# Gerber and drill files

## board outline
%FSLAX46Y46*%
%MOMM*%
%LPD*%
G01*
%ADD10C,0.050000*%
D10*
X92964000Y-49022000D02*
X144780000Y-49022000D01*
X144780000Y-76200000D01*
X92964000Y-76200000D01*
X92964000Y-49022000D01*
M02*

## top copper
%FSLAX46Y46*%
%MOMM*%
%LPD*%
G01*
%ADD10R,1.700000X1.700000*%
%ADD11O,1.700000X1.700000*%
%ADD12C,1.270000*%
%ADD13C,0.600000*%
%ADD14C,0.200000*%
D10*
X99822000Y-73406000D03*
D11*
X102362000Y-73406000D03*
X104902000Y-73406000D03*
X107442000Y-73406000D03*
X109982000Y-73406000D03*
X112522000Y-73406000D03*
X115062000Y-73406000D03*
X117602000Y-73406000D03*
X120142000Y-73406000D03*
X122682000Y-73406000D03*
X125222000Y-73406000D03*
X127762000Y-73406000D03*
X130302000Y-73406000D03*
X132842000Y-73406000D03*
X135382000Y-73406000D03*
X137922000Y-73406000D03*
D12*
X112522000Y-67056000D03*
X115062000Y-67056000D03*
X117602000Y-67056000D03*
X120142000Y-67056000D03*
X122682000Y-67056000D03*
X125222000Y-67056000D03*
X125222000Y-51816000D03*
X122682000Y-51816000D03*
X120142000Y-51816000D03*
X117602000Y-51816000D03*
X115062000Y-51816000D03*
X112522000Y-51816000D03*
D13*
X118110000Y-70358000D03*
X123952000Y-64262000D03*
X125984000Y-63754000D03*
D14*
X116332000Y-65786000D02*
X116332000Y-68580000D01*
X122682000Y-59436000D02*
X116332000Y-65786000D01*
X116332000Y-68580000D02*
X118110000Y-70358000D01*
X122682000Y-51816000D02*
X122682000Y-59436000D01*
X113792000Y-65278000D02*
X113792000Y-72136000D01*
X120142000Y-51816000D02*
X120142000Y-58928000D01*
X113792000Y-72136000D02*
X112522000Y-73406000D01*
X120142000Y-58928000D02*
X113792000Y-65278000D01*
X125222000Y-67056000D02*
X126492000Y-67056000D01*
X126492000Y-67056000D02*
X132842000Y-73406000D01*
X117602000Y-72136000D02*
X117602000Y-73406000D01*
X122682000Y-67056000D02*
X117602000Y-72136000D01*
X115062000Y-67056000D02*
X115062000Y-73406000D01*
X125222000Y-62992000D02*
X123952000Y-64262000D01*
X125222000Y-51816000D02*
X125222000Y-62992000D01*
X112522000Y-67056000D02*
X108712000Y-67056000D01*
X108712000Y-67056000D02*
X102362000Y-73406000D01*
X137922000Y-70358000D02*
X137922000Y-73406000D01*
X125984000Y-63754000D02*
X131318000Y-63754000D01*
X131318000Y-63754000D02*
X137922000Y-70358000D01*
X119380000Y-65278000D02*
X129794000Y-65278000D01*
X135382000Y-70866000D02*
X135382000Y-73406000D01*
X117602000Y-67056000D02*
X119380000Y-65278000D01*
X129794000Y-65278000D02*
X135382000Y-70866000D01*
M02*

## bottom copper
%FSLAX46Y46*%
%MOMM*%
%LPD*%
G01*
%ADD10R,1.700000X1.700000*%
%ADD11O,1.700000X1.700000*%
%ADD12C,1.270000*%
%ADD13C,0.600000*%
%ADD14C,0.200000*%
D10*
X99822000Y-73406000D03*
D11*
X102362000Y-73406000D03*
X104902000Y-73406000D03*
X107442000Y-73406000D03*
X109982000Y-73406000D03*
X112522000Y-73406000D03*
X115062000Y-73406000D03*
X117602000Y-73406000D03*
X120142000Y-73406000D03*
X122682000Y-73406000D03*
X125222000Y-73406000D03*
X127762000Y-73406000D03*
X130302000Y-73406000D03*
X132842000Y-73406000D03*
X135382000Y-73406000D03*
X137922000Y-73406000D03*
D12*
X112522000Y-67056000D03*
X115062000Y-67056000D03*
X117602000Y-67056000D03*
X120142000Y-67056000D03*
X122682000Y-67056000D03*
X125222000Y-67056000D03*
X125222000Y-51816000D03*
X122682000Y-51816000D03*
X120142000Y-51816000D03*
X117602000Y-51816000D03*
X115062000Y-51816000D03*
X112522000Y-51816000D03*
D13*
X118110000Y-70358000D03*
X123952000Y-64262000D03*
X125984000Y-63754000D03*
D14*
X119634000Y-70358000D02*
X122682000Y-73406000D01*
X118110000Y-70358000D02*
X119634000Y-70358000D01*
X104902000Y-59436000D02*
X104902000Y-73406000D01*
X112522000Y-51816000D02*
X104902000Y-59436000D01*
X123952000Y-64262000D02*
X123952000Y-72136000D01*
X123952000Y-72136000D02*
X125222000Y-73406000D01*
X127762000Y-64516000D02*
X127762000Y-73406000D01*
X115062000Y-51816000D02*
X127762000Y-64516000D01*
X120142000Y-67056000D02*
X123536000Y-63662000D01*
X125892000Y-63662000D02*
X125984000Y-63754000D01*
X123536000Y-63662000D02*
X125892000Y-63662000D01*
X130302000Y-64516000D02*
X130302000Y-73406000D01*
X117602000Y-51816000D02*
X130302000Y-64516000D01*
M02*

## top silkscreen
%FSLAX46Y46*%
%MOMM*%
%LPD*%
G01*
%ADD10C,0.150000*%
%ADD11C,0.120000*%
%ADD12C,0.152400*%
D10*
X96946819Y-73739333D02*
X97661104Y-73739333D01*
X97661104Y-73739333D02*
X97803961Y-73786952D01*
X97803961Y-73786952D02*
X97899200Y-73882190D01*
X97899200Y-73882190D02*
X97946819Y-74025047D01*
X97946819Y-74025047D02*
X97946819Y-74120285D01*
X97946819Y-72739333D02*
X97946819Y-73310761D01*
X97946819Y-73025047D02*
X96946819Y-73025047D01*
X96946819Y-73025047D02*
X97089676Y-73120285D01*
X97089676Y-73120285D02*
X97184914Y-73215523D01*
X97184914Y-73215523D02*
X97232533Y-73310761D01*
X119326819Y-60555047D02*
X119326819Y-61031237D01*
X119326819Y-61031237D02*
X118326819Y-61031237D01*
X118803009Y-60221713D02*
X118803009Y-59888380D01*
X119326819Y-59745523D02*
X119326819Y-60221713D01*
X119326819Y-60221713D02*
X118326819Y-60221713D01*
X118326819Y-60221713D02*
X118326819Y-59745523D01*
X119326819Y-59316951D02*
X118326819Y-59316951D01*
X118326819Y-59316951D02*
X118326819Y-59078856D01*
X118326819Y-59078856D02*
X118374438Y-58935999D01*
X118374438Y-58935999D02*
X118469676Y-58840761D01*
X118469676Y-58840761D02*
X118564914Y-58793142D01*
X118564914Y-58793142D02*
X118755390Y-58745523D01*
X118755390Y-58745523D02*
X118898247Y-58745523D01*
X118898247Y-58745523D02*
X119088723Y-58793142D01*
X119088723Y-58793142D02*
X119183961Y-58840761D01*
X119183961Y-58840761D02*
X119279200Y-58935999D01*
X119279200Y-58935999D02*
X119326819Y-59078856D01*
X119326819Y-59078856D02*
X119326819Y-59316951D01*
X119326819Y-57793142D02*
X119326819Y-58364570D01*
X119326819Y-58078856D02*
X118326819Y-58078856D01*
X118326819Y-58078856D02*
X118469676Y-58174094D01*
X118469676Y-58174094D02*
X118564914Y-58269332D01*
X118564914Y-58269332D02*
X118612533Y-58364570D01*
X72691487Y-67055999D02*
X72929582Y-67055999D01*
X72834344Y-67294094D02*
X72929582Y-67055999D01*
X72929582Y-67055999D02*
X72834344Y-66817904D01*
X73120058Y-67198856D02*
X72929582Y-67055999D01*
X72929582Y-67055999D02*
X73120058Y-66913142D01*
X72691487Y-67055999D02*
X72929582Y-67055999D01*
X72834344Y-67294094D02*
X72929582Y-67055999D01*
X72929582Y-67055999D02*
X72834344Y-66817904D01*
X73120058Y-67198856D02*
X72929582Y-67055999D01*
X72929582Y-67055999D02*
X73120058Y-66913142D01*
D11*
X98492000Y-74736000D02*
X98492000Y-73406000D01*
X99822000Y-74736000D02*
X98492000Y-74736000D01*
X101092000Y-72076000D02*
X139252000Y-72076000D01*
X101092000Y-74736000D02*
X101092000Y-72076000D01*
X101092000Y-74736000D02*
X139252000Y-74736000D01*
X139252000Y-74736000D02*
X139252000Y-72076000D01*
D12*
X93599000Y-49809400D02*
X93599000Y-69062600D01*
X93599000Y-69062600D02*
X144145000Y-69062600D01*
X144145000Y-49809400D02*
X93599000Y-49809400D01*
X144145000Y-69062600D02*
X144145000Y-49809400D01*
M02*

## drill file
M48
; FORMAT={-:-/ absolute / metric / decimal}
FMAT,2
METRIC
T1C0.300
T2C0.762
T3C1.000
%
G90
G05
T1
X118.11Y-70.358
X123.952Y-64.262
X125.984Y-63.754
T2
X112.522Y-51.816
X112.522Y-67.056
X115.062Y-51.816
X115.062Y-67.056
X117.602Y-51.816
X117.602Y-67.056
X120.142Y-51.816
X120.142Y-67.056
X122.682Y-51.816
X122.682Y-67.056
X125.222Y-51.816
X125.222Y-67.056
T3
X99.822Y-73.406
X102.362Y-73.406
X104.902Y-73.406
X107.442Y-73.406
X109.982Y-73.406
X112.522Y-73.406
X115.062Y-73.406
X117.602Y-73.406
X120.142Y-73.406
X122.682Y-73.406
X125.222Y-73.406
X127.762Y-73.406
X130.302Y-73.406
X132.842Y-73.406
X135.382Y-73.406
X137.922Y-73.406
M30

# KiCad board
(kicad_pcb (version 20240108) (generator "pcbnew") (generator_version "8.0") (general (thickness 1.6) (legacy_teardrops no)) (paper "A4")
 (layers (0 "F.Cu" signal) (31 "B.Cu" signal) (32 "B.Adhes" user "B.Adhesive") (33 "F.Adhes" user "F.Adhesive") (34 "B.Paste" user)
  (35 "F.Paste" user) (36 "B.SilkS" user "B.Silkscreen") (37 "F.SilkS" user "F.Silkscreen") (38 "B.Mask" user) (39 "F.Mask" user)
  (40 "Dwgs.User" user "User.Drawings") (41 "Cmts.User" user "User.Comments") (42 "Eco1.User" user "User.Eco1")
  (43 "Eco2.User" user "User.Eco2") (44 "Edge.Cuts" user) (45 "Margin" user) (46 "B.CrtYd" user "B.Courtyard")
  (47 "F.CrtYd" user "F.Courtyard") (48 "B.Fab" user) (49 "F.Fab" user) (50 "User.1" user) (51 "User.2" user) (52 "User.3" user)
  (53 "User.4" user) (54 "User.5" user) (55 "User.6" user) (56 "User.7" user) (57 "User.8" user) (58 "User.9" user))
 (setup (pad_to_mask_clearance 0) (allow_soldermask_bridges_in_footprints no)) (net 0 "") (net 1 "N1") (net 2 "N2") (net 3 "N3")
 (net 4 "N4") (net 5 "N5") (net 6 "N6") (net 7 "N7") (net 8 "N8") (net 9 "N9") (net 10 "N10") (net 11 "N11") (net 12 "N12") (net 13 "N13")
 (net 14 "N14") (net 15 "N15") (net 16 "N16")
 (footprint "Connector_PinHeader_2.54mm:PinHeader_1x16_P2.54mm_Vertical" (layer "F.Cu") (at 99.822 73.406 90)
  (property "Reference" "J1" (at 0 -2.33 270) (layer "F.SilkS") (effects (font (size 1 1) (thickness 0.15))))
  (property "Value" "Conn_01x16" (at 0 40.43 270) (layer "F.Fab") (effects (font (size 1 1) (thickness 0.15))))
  (fp_line (start -1.33 -1.33) (end 0 -1.33) (stroke (width 0.12) (type solid)) (layer "F.SilkS"))
  (fp_line (start -1.33 0) (end -1.33 -1.33) (stroke (width 0.12) (type solid)) (layer "F.SilkS"))
  (fp_line (start 1.33 1.27) (end 1.33 39.43) (stroke (width 0.12) (type solid)) (layer "F.SilkS"))
  (fp_line (start -1.33 1.27) (end 1.33 1.27) (stroke (width 0.12) (type solid)) (layer "F.SilkS"))
  (fp_line (start -1.33 1.27) (end -1.33 39.43) (stroke (width 0.12) (type solid)) (layer "F.SilkS"))
  (fp_line (start -1.33 39.43) (end 1.33 39.43) (stroke (width 0.12) (type solid)) (layer "F.SilkS"))
  (pad "1" thru_hole rect (at 0 0 90) (size 1.7 1.7) (drill 1) (layers "*.Cu" "*.Mask") (remove_unused_layers no) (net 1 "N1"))
  (pad "2" thru_hole oval (at 0 2.54 90) (size 1.7 1.7) (drill 1) (layers "*.Cu" "*.Mask") (remove_unused_layers no) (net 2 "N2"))
  (pad "3" thru_hole oval (at 0 5.08 90) (size 1.7 1.7) (drill 1) (layers "*.Cu" "*.Mask") (remove_unused_layers no) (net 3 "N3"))
  (pad "4" thru_hole oval (at 0 7.62 90) (size 1.7 1.7) (drill 1) (layers "*.Cu" "*.Mask") (remove_unused_layers no) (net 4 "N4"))
  (pad "5" thru_hole oval (at 0 10.16 90) (size 1.7 1.7) (drill 1) (layers "*.Cu" "*.Mask") (remove_unused_layers no) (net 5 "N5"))
  (pad "6" thru_hole oval (at 0 12.7 90) (size 1.7 1.7) (drill 1) (layers "*.Cu" "*.Mask") (remove_unused_layers no) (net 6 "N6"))
  (pad "7" thru_hole oval (at 0 15.24 90) (size 1.7 1.7) (drill 1) (layers "*.Cu" "*.Mask") (remove_unused_layers no) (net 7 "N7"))
  (pad "8" thru_hole oval (at 0 17.78 90) (size 1.7 1.7) (drill 1) (layers "*.Cu" "*.Mask") (remove_unused_layers no) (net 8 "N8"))
  (pad "9" thru_hole oval (at 0 20.32 90) (size 1.7 1.7) (drill 1) (layers "*.Cu" "*.Mask") (remove_unused_layers no) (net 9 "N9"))
  (pad "10" thru_hole oval (at 0 22.86 90) (size 1.7 1.7) (drill 1) (layers "*.Cu" "*.Mask") (remove_unused_layers no) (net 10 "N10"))
  (pad "11" thru_hole oval (at 0 25.4 90) (size 1.7 1.7) (drill 1) (layers "*.Cu" "*.Mask") (remove_unused_layers no) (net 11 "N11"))
  (pad "12" thru_hole oval (at 0 27.94 90) (size 1.7 1.7) (drill 1) (layers "*.Cu" "*.Mask") (remove_unused_layers no) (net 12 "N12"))
  (pad "13" thru_hole oval (at 0 30.48 90) (size 1.7 1.7) (drill 1) (layers "*.Cu" "*.Mask") (remove_unused_layers no) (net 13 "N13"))
  (pad "14" thru_hole oval (at 0 33.02 90) (size 1.7 1.7) (drill 1) (layers "*.Cu" "*.Mask") (remove_unused_layers no) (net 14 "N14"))
  (pad "15" thru_hole oval (at 0 35.56 90) (size 1.7 1.7) (drill 1) (layers "*.Cu" "*.Mask") (remove_unused_layers no) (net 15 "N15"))
  (pad "16" thru_hole oval (at 0 38.1 90) (size 1.7 1.7) (drill 1) (layers "*.Cu" "*.Mask") (remove_unused_layers no) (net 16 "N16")))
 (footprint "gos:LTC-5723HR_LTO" (layer "F.Cu") (at 112.522 67.056 90)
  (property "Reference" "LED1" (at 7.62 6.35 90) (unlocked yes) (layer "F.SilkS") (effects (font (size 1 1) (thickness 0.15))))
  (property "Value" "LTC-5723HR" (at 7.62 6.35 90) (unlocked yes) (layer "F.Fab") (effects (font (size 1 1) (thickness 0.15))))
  (fp_line (start 17.2466 -18.923) (end -2.0066 -18.923) (stroke (width 0.1524) (type solid)) (layer "F.SilkS"))
  (fp_line (start -2.0066 -18.923) (end -2.0066 31.623) (stroke (width 0.1524) (type solid)) (layer "F.SilkS"))
  (fp_line (start 17.2466 31.623) (end 17.2466 -18.923) (stroke (width 0.1524) (type solid)) (layer "F.SilkS"))
  (fp_line (start -2.0066 31.623) (end 17.2466 31.623) (stroke (width 0.1524) (type solid)) (layer "F.SilkS"))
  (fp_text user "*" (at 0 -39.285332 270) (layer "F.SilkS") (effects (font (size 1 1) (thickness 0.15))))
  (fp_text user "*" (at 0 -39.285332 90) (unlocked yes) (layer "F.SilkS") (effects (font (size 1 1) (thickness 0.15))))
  (pad "1" thru_hole circle (at 0 0 90) (size 1.27 1.27) (drill 0.762) (layers "*.Cu" "*.Mask") (remove_unused_layers no) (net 2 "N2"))
  (pad "2" thru_hole circle (at 0 2.54 90) (size 1.27 1.27) (drill 0.762) (layers "*.Cu" "*.Mask") (remove_unused_layers no) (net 7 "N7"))
  (pad "3" thru_hole circle (at 0 5.08 90) (size 1.27 1.27) (drill 0.762) (layers "*.Cu" "*.Mask") (remove_unused_layers no) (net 15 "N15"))
  (pad "4" thru_hole circle (at 0 7.62 90) (size 1.27 1.27) (drill 0.762) (layers "*.Cu" "*.Mask") (remove_unused_layers no) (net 16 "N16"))
  (pad "5" thru_hole circle (at 0 10.16 90) (size 1.27 1.27) (drill 0.762) (layers "*.Cu" "*.Mask") (remove_unused_layers no) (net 8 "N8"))
  (pad "6" thru_hole circle (at 0 12.7 90) (size 1.27 1.27) (drill 0.762) (layers "*.Cu" "*.Mask") (remove_unused_layers no) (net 14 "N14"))
  (pad "7" thru_hole circle (at 15.24 12.7 90) (size 1.27 1.27) (drill 0.762) (layers "*.Cu" "*.Mask") (remove_unused_layers no)
   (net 11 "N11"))
  (pad "8" thru_hole circle (at 15.24 10.16 90) (size 1.27 1.27) (drill 0.762) (layers "*.Cu" "*.Mask") (remove_unused_layers no)
   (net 10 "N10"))
  (pad "9" thru_hole circle (at 15.24 7.62 90) (size 1.27 1.27) (drill 0.762) (layers "*.Cu" "*.Mask") (remove_unused_layers no)
   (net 6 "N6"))
  (pad "10" thru_hole circle (at 15.24 5.08 90) (size 1.27 1.27) (drill 0.762) (layers "*.Cu" "*.Mask") (remove_unused_layers no)
   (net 13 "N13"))
  (pad "11" thru_hole circle (at 15.24 2.54 90) (size 1.27 1.27) (drill 0.762) (layers "*.Cu" "*.Mask") (remove_unused_layers no)
   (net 12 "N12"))
  (pad "12" thru_hole circle (at 15.24 0 90) (size 1.27 1.27) (drill 0.762) (layers "*.Cu" "*.Mask") (remove_unused_layers no) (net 3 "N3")))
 (gr_rect (start 92.964 49.022) (end 144.78 76.2) (stroke (width 0.05) (type default)) (fill none) (layer "Edge.Cuts"))
 (segment (start 116.332 65.786) (end 116.332 68.58) (width 0.2) (layer "F.Cu") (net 10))
 (segment (start 122.682 59.436) (end 116.332 65.786) (width 0.2) (layer "F.Cu") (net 10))
 (segment (start 116.332 68.58) (end 118.11 70.358) (width 0.2) (layer "F.Cu") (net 10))
 (segment (start 122.682 51.816) (end 122.682 59.436) (width 0.2) (layer "F.Cu") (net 10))
 (via (at 118.11 70.358) (size 0.6) (drill 0.3) (layers "F.Cu" "B.Cu") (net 10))
 (segment (start 119.634 70.358) (end 122.682 73.406) (width 0.2) (layer "B.Cu") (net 10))
 (segment (start 118.11 70.358) (end 119.634 70.358) (width 0.2) (layer "B.Cu") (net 10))
 (segment (start 113.792 65.278) (end 113.792 72.136) (width 0.2) (layer "F.Cu") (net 6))
 (segment (start 120.142 51.816) (end 120.142 58.928) (width 0.2) (layer "F.Cu") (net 6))
 (segment (start 113.792 72.136) (end 112.522 73.406) (width 0.2) (layer "F.Cu") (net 6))
 (segment (start 120.142 58.928) (end 113.792 65.278) (width 0.2) (layer "F.Cu") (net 6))
 (segment (start 125.222 67.056) (end 126.492 67.056) (width 0.2) (layer "F.Cu") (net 14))
 (segment (start 126.492 67.056) (end 132.842 73.406) (width 0.2) (layer "F.Cu") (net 14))
 (segment (start 117.602 72.136) (end 117.602 73.406) (width 0.2) (layer "F.Cu") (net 8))
 (segment (start 122.682 67.056) (end 117.602 72.136) (width 0.2) (layer "F.Cu") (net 8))
 (segment (start 104.902 59.436) (end 104.902 73.406) (width 0.2) (layer "B.Cu") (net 3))
 (segment (start 112.522 51.816) (end 104.902 59.436) (width 0.2) (layer "B.Cu") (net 3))
 (segment (start 115.062 67.056) (end 115.062 73.406) (width 0.2) (layer "F.Cu") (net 7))
 (segment (start 125.222 62.992) (end 123.952 64.262) (width 0.2) (layer "F.Cu") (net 11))
 (segment (start 125.222 51.816) (end 125.222 62.992) (width 0.2) (layer "F.Cu") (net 11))
 (via (at 123.952 64.262) (size 0.6) (drill 0.3) (layers "F.Cu" "B.Cu") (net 11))
 (segment (start 123.952 64.262) (end 123.952 72.136) (width 0.2) (layer "B.Cu") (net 11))
 (segment (start 123.952 72.136) (end 125.222 73.406) (width 0.2) (layer "B.Cu") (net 11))
 (segment (start 112.522 67.056) (end 108.712 67.056) (width 0.2) (layer "F.Cu") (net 2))
 (segment (start 108.712 67.056) (end 102.362 73.406) (width 0.2) (layer "F.Cu") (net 2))
 (segment (start 127.762 64.516) (end 127.762 73.406) (width 0.2) (layer "B.Cu") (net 12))
 (segment (start 115.062 51.816) (end 127.762 64.516) (width 0.2) (layer "B.Cu") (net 12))
 (segment (start 137.922 70.358) (end 137.922 73.406) (width 0.2) (layer "F.Cu") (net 16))
 (segment (start 125.984 63.754) (end 131.318 63.754) (width 0.2) (layer "F.Cu") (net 16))
 (segment (start 131.318 63.754) (end 137.922 70.358) (width 0.2) (layer "F.Cu") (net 16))
 (via (at 125.984 63.754) (size 0.6) (drill 0.3) (layers "F.Cu" "B.Cu") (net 16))
 (segment (start 120.142 67.056) (end 123.536 63.662) (width 0.2) (layer "B.Cu") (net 16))
 (segment (start 125.892 63.662) (end 125.984 63.754) (width 0.2) (layer "B.Cu") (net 16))
 (segment (start 123.536 63.662) (end 125.892 63.662) (width 0.2) (layer "B.Cu") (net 16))
 (segment (start 130.302 64.516) (end 130.302 73.406) (width 0.2) (layer "B.Cu") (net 13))
 (segment (start 117.602 51.816) (end 130.302 64.516) (width 0.2) (layer "B.Cu") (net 13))
 (segment (start 119.38 65.278) (end 129.794 65.278) (width 0.2) (layer "F.Cu") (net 15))
 (segment (start 135.382 70.866) (end 135.382 73.406) (width 0.2) (layer "F.Cu") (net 15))
 (segment (start 117.602 67.056) (end 119.38 65.278) (width 0.2) (layer "F.Cu") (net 15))
 (segment (start 129.794 65.278) (end 135.382 70.866) (width 0.2) (layer "F.Cu") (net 15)))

